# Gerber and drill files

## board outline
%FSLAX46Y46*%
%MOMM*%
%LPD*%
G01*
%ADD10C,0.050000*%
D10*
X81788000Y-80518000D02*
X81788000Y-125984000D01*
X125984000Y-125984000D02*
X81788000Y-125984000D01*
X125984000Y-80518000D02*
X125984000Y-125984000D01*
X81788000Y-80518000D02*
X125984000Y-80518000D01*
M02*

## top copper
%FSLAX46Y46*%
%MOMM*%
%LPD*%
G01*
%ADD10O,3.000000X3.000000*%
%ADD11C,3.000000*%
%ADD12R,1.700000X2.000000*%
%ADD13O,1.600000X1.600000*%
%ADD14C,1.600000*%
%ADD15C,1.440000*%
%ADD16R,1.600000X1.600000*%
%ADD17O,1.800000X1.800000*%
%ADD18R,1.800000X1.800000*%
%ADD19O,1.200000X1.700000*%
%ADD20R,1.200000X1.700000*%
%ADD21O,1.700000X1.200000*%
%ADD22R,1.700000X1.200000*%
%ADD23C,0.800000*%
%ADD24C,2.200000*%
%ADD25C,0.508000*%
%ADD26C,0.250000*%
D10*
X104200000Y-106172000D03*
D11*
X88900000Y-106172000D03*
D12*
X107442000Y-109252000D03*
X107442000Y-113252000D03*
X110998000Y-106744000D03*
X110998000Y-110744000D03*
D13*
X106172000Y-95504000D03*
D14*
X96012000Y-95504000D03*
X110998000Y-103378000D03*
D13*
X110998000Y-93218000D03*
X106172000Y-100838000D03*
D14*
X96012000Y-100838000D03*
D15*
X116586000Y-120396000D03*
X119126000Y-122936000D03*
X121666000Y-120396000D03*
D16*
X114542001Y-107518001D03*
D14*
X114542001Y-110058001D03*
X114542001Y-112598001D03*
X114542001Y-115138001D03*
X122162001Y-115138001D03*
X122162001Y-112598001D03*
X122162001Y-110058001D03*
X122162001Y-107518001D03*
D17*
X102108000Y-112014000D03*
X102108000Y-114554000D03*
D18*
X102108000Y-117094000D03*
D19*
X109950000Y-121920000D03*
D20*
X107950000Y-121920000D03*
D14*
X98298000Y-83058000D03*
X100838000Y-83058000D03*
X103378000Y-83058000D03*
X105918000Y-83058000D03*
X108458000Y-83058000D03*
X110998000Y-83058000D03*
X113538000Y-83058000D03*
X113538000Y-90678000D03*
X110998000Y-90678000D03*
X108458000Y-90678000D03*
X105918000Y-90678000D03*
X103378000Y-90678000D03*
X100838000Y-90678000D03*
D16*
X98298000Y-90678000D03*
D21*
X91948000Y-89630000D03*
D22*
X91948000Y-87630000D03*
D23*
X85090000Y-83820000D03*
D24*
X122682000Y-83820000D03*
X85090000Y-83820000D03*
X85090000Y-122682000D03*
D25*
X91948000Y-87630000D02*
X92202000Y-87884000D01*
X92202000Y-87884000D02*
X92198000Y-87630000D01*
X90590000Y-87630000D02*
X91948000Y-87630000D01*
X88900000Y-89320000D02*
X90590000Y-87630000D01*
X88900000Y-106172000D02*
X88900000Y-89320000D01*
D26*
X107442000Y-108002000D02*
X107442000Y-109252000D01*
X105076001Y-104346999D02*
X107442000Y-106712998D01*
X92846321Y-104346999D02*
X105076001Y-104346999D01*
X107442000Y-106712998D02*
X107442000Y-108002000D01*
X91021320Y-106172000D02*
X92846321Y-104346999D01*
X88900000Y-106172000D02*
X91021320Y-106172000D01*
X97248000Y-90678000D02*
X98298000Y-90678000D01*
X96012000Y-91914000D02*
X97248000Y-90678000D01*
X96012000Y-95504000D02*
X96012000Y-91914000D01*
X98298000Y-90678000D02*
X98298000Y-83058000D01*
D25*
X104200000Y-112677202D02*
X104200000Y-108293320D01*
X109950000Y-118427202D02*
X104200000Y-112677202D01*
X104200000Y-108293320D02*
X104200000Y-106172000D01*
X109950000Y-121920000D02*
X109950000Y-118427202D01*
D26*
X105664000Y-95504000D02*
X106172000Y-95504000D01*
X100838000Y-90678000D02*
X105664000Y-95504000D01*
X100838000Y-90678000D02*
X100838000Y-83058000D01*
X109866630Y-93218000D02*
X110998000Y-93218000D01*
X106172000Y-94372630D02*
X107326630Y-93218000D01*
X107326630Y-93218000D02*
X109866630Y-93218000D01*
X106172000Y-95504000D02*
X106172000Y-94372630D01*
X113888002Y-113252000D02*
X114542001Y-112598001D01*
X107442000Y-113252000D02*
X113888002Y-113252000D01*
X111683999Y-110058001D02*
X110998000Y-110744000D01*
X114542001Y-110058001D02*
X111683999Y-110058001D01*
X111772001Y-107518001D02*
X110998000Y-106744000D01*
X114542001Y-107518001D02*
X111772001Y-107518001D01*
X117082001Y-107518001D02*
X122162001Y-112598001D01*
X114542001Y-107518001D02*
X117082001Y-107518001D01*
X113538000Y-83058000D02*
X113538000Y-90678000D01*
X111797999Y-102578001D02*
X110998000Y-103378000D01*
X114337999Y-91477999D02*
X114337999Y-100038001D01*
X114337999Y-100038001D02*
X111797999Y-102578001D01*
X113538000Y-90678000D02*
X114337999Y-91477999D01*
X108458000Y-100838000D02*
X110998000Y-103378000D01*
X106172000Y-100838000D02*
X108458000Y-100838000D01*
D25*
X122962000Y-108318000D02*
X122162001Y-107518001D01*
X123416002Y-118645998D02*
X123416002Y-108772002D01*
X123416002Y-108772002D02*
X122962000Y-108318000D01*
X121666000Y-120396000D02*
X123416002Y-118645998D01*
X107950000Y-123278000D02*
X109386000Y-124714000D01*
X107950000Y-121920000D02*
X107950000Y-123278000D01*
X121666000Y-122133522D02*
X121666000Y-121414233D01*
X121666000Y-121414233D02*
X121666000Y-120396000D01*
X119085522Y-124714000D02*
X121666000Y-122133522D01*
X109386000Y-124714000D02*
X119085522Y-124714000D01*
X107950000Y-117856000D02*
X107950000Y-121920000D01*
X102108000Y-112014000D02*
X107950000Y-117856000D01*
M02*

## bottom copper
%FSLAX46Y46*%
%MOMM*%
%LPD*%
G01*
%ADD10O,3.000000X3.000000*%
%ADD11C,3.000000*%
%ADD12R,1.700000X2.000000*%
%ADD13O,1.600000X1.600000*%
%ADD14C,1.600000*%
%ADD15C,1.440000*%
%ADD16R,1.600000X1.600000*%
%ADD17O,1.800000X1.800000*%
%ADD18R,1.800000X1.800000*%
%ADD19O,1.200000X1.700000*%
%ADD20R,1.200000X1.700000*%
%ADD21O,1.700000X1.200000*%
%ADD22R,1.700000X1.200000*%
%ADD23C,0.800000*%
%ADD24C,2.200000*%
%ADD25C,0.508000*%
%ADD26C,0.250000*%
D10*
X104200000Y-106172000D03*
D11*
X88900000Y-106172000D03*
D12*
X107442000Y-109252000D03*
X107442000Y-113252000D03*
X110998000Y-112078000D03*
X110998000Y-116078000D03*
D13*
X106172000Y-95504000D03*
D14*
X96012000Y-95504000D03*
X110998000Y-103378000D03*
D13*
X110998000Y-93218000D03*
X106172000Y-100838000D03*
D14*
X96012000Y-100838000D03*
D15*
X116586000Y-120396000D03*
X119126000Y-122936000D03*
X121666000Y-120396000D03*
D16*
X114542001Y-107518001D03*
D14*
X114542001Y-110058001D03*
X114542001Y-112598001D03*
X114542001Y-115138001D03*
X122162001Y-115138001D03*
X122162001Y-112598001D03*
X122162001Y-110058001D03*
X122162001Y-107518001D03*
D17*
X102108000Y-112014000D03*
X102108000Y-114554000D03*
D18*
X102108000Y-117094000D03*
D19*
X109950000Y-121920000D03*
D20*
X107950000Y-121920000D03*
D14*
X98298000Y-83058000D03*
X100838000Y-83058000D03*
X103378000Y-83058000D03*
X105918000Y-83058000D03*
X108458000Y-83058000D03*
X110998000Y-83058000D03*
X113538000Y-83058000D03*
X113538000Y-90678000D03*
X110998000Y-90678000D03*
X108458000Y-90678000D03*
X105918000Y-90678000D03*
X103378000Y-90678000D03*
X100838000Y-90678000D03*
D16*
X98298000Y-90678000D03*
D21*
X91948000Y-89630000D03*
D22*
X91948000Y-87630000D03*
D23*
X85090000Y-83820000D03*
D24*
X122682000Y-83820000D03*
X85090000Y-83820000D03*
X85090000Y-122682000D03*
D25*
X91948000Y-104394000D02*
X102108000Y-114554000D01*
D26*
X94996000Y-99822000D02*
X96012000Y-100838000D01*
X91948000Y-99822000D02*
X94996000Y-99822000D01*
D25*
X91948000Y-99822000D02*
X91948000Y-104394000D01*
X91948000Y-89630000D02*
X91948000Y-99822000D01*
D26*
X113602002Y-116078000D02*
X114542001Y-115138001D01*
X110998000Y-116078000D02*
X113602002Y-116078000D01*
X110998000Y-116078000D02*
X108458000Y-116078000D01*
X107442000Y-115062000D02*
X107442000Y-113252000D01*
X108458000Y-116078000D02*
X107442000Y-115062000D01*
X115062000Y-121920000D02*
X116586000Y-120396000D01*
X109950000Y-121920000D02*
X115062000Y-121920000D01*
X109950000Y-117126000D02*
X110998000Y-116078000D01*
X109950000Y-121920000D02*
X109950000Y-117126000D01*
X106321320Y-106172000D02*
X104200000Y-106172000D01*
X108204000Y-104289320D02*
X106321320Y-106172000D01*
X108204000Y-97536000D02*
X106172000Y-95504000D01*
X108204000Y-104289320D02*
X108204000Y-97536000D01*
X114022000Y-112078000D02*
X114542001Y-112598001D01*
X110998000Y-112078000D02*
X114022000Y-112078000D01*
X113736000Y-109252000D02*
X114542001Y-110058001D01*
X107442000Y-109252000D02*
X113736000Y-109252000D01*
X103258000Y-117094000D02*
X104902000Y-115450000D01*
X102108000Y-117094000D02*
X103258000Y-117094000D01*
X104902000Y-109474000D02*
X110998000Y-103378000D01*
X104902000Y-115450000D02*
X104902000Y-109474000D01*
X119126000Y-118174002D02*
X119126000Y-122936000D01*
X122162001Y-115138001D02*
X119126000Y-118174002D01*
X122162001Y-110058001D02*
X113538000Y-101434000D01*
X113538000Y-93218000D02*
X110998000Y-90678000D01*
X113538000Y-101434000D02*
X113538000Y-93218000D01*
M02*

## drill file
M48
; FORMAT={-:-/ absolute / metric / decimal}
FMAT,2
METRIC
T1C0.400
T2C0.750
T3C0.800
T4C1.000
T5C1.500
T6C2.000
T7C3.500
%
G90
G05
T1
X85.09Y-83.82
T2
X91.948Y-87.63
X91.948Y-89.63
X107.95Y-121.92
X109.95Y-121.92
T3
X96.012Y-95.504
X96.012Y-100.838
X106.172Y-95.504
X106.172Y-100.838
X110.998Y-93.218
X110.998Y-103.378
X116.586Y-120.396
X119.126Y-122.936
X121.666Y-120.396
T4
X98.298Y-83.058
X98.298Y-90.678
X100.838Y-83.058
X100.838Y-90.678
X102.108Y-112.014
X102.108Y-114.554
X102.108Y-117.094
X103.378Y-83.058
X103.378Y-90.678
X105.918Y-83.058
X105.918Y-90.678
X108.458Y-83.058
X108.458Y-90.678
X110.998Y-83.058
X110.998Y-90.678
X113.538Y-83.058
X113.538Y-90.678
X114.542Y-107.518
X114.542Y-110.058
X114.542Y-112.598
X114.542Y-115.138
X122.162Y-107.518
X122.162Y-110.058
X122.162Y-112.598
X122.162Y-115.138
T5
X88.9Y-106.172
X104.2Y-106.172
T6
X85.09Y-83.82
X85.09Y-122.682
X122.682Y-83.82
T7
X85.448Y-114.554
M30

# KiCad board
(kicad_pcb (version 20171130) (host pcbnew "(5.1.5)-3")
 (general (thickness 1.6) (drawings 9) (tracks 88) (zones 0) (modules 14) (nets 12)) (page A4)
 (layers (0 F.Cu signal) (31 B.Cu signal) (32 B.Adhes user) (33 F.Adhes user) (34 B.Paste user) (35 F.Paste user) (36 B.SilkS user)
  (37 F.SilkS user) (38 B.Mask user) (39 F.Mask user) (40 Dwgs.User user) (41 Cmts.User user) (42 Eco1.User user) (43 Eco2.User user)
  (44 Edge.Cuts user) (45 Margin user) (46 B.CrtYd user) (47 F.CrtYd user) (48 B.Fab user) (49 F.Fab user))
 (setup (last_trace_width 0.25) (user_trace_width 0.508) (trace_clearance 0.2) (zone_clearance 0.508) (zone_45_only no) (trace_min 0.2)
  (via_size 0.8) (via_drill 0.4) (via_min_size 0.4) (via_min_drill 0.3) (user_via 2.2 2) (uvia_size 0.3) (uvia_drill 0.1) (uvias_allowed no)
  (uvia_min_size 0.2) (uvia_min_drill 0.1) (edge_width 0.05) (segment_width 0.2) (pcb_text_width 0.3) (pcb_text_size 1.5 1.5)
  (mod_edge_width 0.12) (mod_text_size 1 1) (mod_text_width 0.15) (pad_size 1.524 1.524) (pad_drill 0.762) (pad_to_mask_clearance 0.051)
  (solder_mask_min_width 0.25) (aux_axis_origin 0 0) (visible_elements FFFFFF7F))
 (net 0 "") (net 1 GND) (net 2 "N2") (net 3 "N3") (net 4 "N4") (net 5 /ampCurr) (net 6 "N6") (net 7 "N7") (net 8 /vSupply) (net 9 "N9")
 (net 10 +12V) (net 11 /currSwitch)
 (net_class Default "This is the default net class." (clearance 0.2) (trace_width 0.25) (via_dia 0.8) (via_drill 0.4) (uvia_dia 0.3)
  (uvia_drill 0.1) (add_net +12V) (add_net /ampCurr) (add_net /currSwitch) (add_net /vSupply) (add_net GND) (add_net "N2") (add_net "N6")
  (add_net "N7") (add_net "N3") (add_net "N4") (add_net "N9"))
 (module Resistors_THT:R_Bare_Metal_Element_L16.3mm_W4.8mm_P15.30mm (layer F.Cu) (at 88.9 106.172)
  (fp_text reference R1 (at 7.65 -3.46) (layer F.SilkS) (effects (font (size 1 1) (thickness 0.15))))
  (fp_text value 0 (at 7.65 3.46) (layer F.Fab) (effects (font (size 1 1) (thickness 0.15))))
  (pad 2 thru_hole oval (at 15.3 0) (size 3 3) (drill 1.5) (layers *.Cu *.Mask) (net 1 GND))
  (pad 1 thru_hole circle (at 0 0) (size 3 3) (drill 1.5) (layers *.Cu *.Mask) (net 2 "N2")))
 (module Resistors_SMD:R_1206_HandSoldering (layer F.Cu) (at 107.442 111.252 90)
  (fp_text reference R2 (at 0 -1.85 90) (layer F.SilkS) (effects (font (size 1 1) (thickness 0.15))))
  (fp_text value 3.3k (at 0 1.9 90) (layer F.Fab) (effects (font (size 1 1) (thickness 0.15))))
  (pad 2 smd rect (at 2 0 90) (size 2 1.7) (layers F.Cu F.Paste F.Mask) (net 2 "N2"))
  (pad 1 smd rect (at -2 0 90) (size 2 1.7) (layers F.Cu F.Paste F.Mask) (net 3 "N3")))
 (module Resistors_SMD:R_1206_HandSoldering (layer B.Cu) (at 107.442 111.252 270)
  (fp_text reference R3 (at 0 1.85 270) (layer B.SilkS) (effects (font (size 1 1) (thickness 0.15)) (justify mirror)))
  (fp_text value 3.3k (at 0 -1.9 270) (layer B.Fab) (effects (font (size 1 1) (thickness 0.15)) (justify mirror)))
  (pad 1 smd rect (at -2 0 270) (size 2 1.7) (layers B.Cu B.Paste B.Mask) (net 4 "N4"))
  (pad 2 smd rect (at 2 0 270) (size 2 1.7) (layers B.Cu B.Paste B.Mask) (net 1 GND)))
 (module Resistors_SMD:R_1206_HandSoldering (layer B.Cu) (at 110.998 114.078 270)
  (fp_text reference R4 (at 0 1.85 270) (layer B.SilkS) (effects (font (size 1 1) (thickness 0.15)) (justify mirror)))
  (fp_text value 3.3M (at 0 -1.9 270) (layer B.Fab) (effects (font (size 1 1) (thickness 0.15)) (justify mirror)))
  (pad 1 smd rect (at -2 0 270) (size 2 1.7) (layers B.Cu B.Paste B.Mask) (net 3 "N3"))
  (pad 2 smd rect (at 2 0 270) (size 2 1.7) (layers B.Cu B.Paste B.Mask) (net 1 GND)))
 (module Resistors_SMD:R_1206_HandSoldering (layer F.Cu) (at 110.998 108.744 90)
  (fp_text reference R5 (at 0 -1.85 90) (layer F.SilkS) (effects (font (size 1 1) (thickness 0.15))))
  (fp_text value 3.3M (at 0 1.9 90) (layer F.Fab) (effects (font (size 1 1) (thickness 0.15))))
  (pad 2 smd rect (at 2 0 90) (size 2 1.7) (layers F.Cu F.Paste F.Mask) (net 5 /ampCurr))
  (pad 1 smd rect (at -2 0 90) (size 2 1.7) (layers F.Cu F.Paste F.Mask) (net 4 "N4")))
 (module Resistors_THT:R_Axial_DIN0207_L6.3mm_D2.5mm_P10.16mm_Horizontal (layer F.Cu) (at 96.012 95.504)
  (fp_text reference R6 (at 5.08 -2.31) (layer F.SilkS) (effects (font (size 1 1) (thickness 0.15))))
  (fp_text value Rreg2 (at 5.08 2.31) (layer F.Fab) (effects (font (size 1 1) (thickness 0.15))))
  (pad 2 thru_hole oval (at 10.16 0) (size 1.6 1.6) (drill 0.8) (layers *.Cu *.Mask) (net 1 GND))
  (pad 1 thru_hole circle (at 0 0) (size 1.6 1.6) (drill 0.8) (layers *.Cu *.Mask) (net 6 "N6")))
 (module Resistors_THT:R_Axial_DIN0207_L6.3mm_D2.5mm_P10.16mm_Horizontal (layer F.Cu) (at 110.998 103.378 90)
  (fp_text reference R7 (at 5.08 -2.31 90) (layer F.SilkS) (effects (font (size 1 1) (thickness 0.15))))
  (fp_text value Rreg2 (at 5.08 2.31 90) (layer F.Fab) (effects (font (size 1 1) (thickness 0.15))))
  (pad 1 thru_hole circle (at 0 0 90) (size 1.6 1.6) (drill 0.8) (layers *.Cu *.Mask) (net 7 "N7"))
  (pad 2 thru_hole oval (at 10.16 0 90) (size 1.6 1.6) (drill 0.8) (layers *.Cu *.Mask) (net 1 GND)))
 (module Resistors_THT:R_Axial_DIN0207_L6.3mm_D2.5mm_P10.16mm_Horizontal (layer F.Cu) (at 96.012 100.838)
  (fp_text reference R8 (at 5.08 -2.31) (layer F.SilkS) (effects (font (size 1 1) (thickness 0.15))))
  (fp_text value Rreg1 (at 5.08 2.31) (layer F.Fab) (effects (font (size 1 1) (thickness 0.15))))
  (pad 2 thru_hole oval (at 10.16 0) (size 1.6 1.6) (drill 0.8) (layers *.Cu *.Mask) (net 7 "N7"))
  (pad 1 thru_hole circle (at 0 0) (size 1.6 1.6) (drill 0.8) (layers *.Cu *.Mask) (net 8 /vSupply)))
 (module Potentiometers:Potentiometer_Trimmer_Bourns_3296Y (layer F.Cu) (at 121.666 120.396)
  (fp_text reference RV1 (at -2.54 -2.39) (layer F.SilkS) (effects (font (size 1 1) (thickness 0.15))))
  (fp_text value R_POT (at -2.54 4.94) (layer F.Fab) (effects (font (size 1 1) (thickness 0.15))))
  (pad 3 thru_hole circle (at -5.08 0) (size 1.44 1.44) (drill 0.8) (layers *.Cu *.Mask) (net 1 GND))
  (pad 2 thru_hole circle (at -2.54 2.54) (size 1.44 1.44) (drill 0.8) (layers *.Cu *.Mask) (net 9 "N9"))
  (pad 1 thru_hole circle (at 0 0) (size 1.44 1.44) (drill 0.8) (layers *.Cu *.Mask) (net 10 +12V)))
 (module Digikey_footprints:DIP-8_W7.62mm (layer F.Cu) (at 114.542001 107.518001)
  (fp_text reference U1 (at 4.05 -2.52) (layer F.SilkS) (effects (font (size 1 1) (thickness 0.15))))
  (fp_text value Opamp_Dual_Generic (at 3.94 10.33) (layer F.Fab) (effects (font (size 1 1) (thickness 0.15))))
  (pad 1 thru_hole rect (at 0 0) (size 1.6 1.6) (drill 1) (layers *.Cu *.Mask) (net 5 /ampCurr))
  (pad 2 thru_hole circle (at 0 2.54) (size 1.6 1.6) (drill 1) (layers *.Cu *.Mask) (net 4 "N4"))
  (pad 3 thru_hole circle (at 0 5.08) (size 1.6 1.6) (drill 1) (layers *.Cu *.Mask) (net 3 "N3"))
  (pad 4 thru_hole circle (at 0 7.62) (size 1.6 1.6) (drill 1) (layers *.Cu *.Mask) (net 1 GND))
  (pad 5 thru_hole circle (at 7.62 7.62) (size 1.6 1.6) (drill 1) (layers *.Cu *.Mask) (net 9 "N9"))
  (pad 6 thru_hole circle (at 7.62 5.08) (size 1.6 1.6) (drill 1) (layers *.Cu *.Mask) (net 5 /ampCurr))
  (pad 7 thru_hole circle (at 7.62 2.54) (size 1.6 1.6) (drill 1) (layers *.Cu *.Mask) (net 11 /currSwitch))
  (pad 8 thru_hole circle (at 7.62 0) (size 1.6 1.6) (drill 1) (layers *.Cu *.Mask) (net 10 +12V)))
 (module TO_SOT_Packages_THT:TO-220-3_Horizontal (layer F.Cu) (at 102.108 117.094 90)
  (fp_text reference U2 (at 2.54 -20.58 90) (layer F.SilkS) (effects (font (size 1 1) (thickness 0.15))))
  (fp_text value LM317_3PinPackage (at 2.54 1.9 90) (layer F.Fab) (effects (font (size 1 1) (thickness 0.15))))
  (pad 3 thru_hole oval (at 5.08 0 90) (size 1.8 1.8) (drill 1) (layers *.Cu *.Mask) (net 10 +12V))
  (pad 2 thru_hole oval (at 2.54 0 90) (size 1.8 1.8) (drill 1) (layers *.Cu *.Mask) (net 8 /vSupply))
  (pad 1 thru_hole rect (at 0 0 90) (size 1.8 1.8) (drill 1) (layers *.Cu *.Mask) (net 7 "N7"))
  (pad 0 np_thru_hole oval (at 2.54 -16.66 90) (size 3.5 3.5) (drill 3.5) (layers *.Cu *.Mask)))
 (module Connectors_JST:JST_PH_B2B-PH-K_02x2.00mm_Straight (layer F.Cu) (at 107.95 121.92)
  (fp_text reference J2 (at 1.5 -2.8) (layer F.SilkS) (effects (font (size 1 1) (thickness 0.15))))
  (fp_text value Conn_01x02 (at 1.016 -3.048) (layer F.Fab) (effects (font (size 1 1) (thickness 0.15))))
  (pad 2 thru_hole oval (at 2 0) (size 1.2 1.7) (drill 0.75) (layers *.Cu *.Mask) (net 1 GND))
  (pad 1 thru_hole rect (at 0 0) (size 1.2 1.7) (drill 0.75) (layers *.Cu *.Mask) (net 10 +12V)))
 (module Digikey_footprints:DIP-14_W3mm (layer F.Cu) (at 98.298 90.678 90)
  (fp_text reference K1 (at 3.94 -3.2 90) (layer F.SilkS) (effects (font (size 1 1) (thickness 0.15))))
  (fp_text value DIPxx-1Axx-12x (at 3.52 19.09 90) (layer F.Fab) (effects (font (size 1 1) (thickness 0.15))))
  (pad 14 thru_hole circle (at 7.62 0 90) (size 1.6 1.6) (drill 1) (layers *.Cu *.Mask) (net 6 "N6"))
  (pad 13 thru_hole circle (at 7.62 2.54 90) (size 1.6 1.6) (drill 1) (layers *.Cu *.Mask) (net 1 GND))
  (pad 12 thru_hole circle (at 7.62 5.08 90) (size 1.6 1.6) (drill 1) (layers *.Cu *.Mask))
  (pad 11 thru_hole circle (at 7.62 7.62 90) (size 1.6 1.6) (drill 1) (layers *.Cu *.Mask))
  (pad 10 thru_hole circle (at 7.62 10.16 90) (size 1.6 1.6) (drill 1) (layers *.Cu *.Mask))
  (pad 9 thru_hole circle (at 7.62 12.7 90) (size 1.6 1.6) (drill 1) (layers *.Cu *.Mask))
  (pad 8 thru_hole circle (at 7.62 15.24 90) (size 1.6 1.6) (drill 1) (layers *.Cu *.Mask) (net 7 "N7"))
  (pad 7 thru_hole circle (at 0 15.24 90) (size 1.6 1.6) (drill 1) (layers *.Cu *.Mask) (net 7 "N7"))
  (pad 6 thru_hole circle (at 0 12.7 90) (size 1.6 1.6) (drill 1) (layers *.Cu *.Mask) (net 11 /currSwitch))
  (pad 5 thru_hole circle (at 0 10.16 90) (size 1.6 1.6) (drill 1) (layers *.Cu *.Mask))
  (pad 4 thru_hole circle (at 0 7.62 90) (size 1.6 1.6) (drill 1) (layers *.Cu *.Mask))
  (pad 3 thru_hole circle (at 0 5.08 90) (size 1.6 1.6) (drill 1) (layers *.Cu *.Mask))
  (pad 2 thru_hole circle (at 0 2.54 90) (size 1.6 1.6) (drill 1) (layers *.Cu *.Mask) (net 1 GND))
  (pad 1 thru_hole rect (at 0 0 90) (size 1.6 1.6) (drill 1) (layers *.Cu *.Mask) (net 6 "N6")))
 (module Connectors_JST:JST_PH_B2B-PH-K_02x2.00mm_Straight (layer F.Cu) (at 91.948 87.63 270)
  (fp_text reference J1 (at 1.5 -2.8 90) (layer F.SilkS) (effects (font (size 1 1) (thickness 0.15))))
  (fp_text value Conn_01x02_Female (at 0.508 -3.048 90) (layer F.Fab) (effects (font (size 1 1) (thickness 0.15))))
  (pad 2 thru_hole oval (at 2 0 270) (size 1.2 1.7) (drill 0.75) (layers *.Cu *.Mask) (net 8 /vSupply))
  (pad 1 thru_hole rect (at 0 0 270) (size 1.2 1.7) (drill 0.75) (layers *.Cu *.Mask) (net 2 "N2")))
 (gr_line (start 81.788 80.518) (end 81.788 125.984) (layer Edge.Cuts) (width 0.05))
 (gr_line (start 125.984 125.984) (end 81.788 125.984) (layer Edge.Cuts) (width 0.05))
 (gr_line (start 125.984 80.518) (end 125.984 125.984) (layer Edge.Cuts) (width 0.05))
 (gr_line (start 81.788 80.518) (end 125.984 80.518) (layer Edge.Cuts) (width 0.05))
 (via (at 85.09 83.82) (size 0.8) (drill 0.4) (layers F.Cu B.Cu) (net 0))
 (via (at 122.682 83.82) (size 2.2) (drill 2) (layers F.Cu B.Cu) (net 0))
 (via (at 85.09 83.82) (size 2.2) (drill 2) (layers F.Cu B.Cu) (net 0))
 (via (at 85.09 122.682) (size 2.2) (drill 2) (layers F.Cu B.Cu) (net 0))
 (segment (start 91.948 104.394) (end 102.108 114.554) (width 0.508) (layer B.Cu) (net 8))
 (segment (start 94.996 99.822) (end 96.012 100.838) (width 0.25) (layer B.Cu) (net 8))
 (segment (start 91.948 99.822) (end 94.996 99.822) (width 0.25) (layer B.Cu) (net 8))
 (segment (start 91.948 99.822) (end 91.948 104.394) (width 0.508) (layer B.Cu) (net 8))
 (segment (start 91.948 89.63) (end 91.948 99.822) (width 0.508) (layer B.Cu) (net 8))
 (segment (start 91.948 87.63) (end 92.202 87.884) (width 0.508) (layer F.Cu) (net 2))
 (segment (start 92.202 87.884) (end 92.198 87.63) (width 0.508) (layer F.Cu) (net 2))
 (segment (start 90.59 87.63) (end 91.948 87.63) (width 0.508) (layer F.Cu) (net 2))
 (segment (start 88.9 89.32) (end 90.59 87.63) (width 0.508) (layer F.Cu) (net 2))
 (segment (start 88.9 106.172) (end 88.9 89.32) (width 0.508) (layer F.Cu) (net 2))
 (segment (start 107.442 108.002) (end 107.442 109.252) (width 0.25) (layer F.Cu) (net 2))
 (segment (start 105.076001 104.346999) (end 107.442 106.712998) (width 0.25) (layer F.Cu) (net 2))
 (segment (start 92.846321 104.346999) (end 105.076001 104.346999) (width 0.25) (layer F.Cu) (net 2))
 (segment (start 107.442 106.712998) (end 107.442 108.002) (width 0.25) (layer F.Cu) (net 2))
 (segment (start 91.02132 106.172) (end 92.846321 104.346999) (width 0.25) (layer F.Cu) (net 2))
 (segment (start 88.9 106.172) (end 91.02132 106.172) (width 0.25) (layer F.Cu) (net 2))
 (segment (start 97.248 90.678) (end 98.298 90.678) (width 0.25) (layer F.Cu) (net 6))
 (segment (start 96.012 91.914) (end 97.248 90.678) (width 0.25) (layer F.Cu) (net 6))
 (segment (start 96.012 95.504) (end 96.012 91.914) (width 0.25) (layer F.Cu) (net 6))
 (segment (start 98.298 90.678) (end 98.298 83.058) (width 0.25) (layer F.Cu) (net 6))
 (segment (start 113.602002 116.078) (end 114.542001 115.138001) (width 0.25) (layer B.Cu) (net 1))
 (segment (start 110.998 116.078) (end 113.602002 116.078) (width 0.25) (layer B.Cu) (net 1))
 (segment (start 110.998 116.078) (end 108.458 116.078) (width 0.25) (layer B.Cu) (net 1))
 (segment (start 107.442 115.062) (end 107.442 113.252) (width 0.25) (layer B.Cu) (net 1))
 (segment (start 108.458 116.078) (end 107.442 115.062) (width 0.25) (layer B.Cu) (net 1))
 (segment (start 104.2 112.677202) (end 104.2 108.29332) (width 0.508) (layer F.Cu) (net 1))
 (segment (start 109.95 118.427202) (end 104.2 112.677202) (width 0.508) (layer F.Cu) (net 1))
 (segment (start 104.2 108.29332) (end 104.2 106.172) (width 0.508) (layer F.Cu) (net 1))
 (segment (start 109.95 121.92) (end 109.95 118.427202) (width 0.508) (layer F.Cu) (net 1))
 (segment (start 115.062 121.92) (end 116.586 120.396) (width 0.25) (layer B.Cu) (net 1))
 (segment (start 109.95 121.92) (end 115.062 121.92) (width 0.25) (layer B.Cu) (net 1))
 (segment (start 109.95 117.126) (end 110.998 116.078) (width 0.25) (layer B.Cu) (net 1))
 (segment (start 109.95 121.92) (end 109.95 117.126) (width 0.25) (layer B.Cu) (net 1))
 (segment (start 105.664 95.504) (end 106.172 95.504) (width 0.25) (layer F.Cu) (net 1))
 (segment (start 100.838 90.678) (end 105.664 95.504) (width 0.25) (layer F.Cu) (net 1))
 (segment (start 100.838 90.678) (end 100.838 83.058) (width 0.25) (layer F.Cu) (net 1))
 (segment (start 109.86663 93.218) (end 110.998 93.218) (width 0.25) (layer F.Cu) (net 1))
 (segment (start 106.172 94.37263) (end 107.32663 93.218) (width 0.25) (layer F.Cu) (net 1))
 (segment (start 107.32663 93.218) (end 109.86663 93.218) (width 0.25) (layer F.Cu) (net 1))
 (segment (start 106.172 95.504) (end 106.172 94.37263) (width 0.25) (layer F.Cu) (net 1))
 (segment (start 106.32132 106.172) (end 104.2 106.172) (width 0.25) (layer B.Cu) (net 1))
 (segment (start 108.204 104.28932) (end 106.32132 106.172) (width 0.25) (layer B.Cu) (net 1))
 (segment (start 108.204 97.536) (end 106.172 95.504) (width 0.25) (layer B.Cu) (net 1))
 (segment (start 108.204 104.28932) (end 108.204 97.536) (width 0.25) (layer B.Cu) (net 1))
 (segment (start 113.888002 113.252) (end 114.542001 112.598001) (width 0.25) (layer F.Cu) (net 3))
 (segment (start 107.442 113.252) (end 113.888002 113.252) (width 0.25) (layer F.Cu) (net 3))
 (segment (start 114.022 112.078) (end 114.542001 112.598001) (width 0.25) (layer B.Cu) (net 3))
 (segment (start 110.998 112.078) (end 114.022 112.078) (width 0.25) (layer B.Cu) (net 3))
 (segment (start 111.683999 110.058001) (end 110.998 110.744) (width 0.25) (layer F.Cu) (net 4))
 (segment (start 114.542001 110.058001) (end 111.683999 110.058001) (width 0.25) (layer F.Cu) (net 4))
 (segment (start 113.736 109.252) (end 114.542001 110.058001) (width 0.25) (layer B.Cu) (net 4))
 (segment (start 107.442 109.252) (end 113.736 109.252) (width 0.25) (layer B.Cu) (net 4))
 (segment (start 111.772001 107.518001) (end 110.998 106.744) (width 0.25) (layer F.Cu) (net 5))
 (segment (start 114.542001 107.518001) (end 111.772001 107.518001) (width 0.25) (layer F.Cu) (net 5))
 (segment (start 117.082001 107.518001) (end 122.162001 112.598001) (width 0.25) (layer F.Cu) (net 5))
 (segment (start 114.542001 107.518001) (end 117.082001 107.518001) (width 0.25) (layer F.Cu) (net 5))
 (segment (start 113.538 83.058) (end 113.538 90.678) (width 0.25) (layer F.Cu) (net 7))
 (segment (start 111.797999 102.578001) (end 110.998 103.378) (width 0.25) (layer F.Cu) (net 7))
 (segment (start 114.337999 91.477999) (end 114.337999 100.038001) (width 0.25) (layer F.Cu) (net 7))
 (segment (start 114.337999 100.038001) (end 111.797999 102.578001) (width 0.25) (layer F.Cu) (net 7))
 (segment (start 113.538 90.678) (end 114.337999 91.477999) (width 0.25) (layer F.Cu) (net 7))
 (segment (start 108.458 100.838) (end 110.998 103.378) (width 0.25) (layer F.Cu) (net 7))
 (segment (start 106.172 100.838) (end 108.458 100.838) (width 0.25) (layer F.Cu) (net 7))
 (segment (start 103.258 117.094) (end 104.902 115.45) (width 0.25) (layer B.Cu) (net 7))
 (segment (start 102.108 117.094) (end 103.258 117.094) (width 0.25) (layer B.Cu) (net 7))
 (segment (start 104.902 109.474) (end 110.998 103.378) (width 0.25) (layer B.Cu) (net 7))
 (segment (start 104.902 115.45) (end 104.902 109.474) (width 0.25) (layer B.Cu) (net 7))
 (segment (start 119.126 118.174002) (end 119.126 122.936) (width 0.25) (layer B.Cu) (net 9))
 (segment (start 122.162001 115.138001) (end 119.126 118.174002) (width 0.25) (layer B.Cu) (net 9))
 (segment (start 122.962 108.318) (end 122.162001 107.518001) (width 0.508) (layer F.Cu) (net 10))
 (segment (start 123.416002 118.645998) (end 123.416002 108.772002) (width 0.508) (layer F.Cu) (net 10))
 (segment (start 123.416002 108.772002) (end 122.962 108.318) (width 0.508) (layer F.Cu) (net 10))
 (segment (start 121.666 120.396) (end 123.416002 118.645998) (width 0.508) (layer F.Cu) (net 10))
 (segment (start 107.95 123.278) (end 109.386 124.714) (width 0.508) (layer F.Cu) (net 10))
 (segment (start 107.95 121.92) (end 107.95 123.278) (width 0.508) (layer F.Cu) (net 10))
 (segment (start 121.666 122.133522) (end 121.666 121.414233) (width 0.508) (layer F.Cu) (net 10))
 (segment (start 121.666 121.414233) (end 121.666 120.396) (width 0.508) (layer F.Cu) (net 10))
 (segment (start 119.085522 124.714) (end 121.666 122.133522) (width 0.508) (layer F.Cu) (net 10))
 (segment (start 109.386 124.714) (end 119.085522 124.714) (width 0.508) (layer F.Cu) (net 10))
 (segment (start 107.95 117.856) (end 107.95 121.92) (width 0.508) (layer F.Cu) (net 10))
 (segment (start 102.108 112.014) (end 107.95 117.856) (width 0.508) (layer F.Cu) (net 10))
 (segment (start 122.162001 110.058001) (end 113.538 101.434) (width 0.25) (layer B.Cu) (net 11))
 (segment (start 113.538 93.218) (end 110.998 90.678) (width 0.25) (layer B.Cu) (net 11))
 (segment (start 113.538 101.434) (end 113.538 93.218) (width 0.25) (layer B.Cu) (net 11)))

